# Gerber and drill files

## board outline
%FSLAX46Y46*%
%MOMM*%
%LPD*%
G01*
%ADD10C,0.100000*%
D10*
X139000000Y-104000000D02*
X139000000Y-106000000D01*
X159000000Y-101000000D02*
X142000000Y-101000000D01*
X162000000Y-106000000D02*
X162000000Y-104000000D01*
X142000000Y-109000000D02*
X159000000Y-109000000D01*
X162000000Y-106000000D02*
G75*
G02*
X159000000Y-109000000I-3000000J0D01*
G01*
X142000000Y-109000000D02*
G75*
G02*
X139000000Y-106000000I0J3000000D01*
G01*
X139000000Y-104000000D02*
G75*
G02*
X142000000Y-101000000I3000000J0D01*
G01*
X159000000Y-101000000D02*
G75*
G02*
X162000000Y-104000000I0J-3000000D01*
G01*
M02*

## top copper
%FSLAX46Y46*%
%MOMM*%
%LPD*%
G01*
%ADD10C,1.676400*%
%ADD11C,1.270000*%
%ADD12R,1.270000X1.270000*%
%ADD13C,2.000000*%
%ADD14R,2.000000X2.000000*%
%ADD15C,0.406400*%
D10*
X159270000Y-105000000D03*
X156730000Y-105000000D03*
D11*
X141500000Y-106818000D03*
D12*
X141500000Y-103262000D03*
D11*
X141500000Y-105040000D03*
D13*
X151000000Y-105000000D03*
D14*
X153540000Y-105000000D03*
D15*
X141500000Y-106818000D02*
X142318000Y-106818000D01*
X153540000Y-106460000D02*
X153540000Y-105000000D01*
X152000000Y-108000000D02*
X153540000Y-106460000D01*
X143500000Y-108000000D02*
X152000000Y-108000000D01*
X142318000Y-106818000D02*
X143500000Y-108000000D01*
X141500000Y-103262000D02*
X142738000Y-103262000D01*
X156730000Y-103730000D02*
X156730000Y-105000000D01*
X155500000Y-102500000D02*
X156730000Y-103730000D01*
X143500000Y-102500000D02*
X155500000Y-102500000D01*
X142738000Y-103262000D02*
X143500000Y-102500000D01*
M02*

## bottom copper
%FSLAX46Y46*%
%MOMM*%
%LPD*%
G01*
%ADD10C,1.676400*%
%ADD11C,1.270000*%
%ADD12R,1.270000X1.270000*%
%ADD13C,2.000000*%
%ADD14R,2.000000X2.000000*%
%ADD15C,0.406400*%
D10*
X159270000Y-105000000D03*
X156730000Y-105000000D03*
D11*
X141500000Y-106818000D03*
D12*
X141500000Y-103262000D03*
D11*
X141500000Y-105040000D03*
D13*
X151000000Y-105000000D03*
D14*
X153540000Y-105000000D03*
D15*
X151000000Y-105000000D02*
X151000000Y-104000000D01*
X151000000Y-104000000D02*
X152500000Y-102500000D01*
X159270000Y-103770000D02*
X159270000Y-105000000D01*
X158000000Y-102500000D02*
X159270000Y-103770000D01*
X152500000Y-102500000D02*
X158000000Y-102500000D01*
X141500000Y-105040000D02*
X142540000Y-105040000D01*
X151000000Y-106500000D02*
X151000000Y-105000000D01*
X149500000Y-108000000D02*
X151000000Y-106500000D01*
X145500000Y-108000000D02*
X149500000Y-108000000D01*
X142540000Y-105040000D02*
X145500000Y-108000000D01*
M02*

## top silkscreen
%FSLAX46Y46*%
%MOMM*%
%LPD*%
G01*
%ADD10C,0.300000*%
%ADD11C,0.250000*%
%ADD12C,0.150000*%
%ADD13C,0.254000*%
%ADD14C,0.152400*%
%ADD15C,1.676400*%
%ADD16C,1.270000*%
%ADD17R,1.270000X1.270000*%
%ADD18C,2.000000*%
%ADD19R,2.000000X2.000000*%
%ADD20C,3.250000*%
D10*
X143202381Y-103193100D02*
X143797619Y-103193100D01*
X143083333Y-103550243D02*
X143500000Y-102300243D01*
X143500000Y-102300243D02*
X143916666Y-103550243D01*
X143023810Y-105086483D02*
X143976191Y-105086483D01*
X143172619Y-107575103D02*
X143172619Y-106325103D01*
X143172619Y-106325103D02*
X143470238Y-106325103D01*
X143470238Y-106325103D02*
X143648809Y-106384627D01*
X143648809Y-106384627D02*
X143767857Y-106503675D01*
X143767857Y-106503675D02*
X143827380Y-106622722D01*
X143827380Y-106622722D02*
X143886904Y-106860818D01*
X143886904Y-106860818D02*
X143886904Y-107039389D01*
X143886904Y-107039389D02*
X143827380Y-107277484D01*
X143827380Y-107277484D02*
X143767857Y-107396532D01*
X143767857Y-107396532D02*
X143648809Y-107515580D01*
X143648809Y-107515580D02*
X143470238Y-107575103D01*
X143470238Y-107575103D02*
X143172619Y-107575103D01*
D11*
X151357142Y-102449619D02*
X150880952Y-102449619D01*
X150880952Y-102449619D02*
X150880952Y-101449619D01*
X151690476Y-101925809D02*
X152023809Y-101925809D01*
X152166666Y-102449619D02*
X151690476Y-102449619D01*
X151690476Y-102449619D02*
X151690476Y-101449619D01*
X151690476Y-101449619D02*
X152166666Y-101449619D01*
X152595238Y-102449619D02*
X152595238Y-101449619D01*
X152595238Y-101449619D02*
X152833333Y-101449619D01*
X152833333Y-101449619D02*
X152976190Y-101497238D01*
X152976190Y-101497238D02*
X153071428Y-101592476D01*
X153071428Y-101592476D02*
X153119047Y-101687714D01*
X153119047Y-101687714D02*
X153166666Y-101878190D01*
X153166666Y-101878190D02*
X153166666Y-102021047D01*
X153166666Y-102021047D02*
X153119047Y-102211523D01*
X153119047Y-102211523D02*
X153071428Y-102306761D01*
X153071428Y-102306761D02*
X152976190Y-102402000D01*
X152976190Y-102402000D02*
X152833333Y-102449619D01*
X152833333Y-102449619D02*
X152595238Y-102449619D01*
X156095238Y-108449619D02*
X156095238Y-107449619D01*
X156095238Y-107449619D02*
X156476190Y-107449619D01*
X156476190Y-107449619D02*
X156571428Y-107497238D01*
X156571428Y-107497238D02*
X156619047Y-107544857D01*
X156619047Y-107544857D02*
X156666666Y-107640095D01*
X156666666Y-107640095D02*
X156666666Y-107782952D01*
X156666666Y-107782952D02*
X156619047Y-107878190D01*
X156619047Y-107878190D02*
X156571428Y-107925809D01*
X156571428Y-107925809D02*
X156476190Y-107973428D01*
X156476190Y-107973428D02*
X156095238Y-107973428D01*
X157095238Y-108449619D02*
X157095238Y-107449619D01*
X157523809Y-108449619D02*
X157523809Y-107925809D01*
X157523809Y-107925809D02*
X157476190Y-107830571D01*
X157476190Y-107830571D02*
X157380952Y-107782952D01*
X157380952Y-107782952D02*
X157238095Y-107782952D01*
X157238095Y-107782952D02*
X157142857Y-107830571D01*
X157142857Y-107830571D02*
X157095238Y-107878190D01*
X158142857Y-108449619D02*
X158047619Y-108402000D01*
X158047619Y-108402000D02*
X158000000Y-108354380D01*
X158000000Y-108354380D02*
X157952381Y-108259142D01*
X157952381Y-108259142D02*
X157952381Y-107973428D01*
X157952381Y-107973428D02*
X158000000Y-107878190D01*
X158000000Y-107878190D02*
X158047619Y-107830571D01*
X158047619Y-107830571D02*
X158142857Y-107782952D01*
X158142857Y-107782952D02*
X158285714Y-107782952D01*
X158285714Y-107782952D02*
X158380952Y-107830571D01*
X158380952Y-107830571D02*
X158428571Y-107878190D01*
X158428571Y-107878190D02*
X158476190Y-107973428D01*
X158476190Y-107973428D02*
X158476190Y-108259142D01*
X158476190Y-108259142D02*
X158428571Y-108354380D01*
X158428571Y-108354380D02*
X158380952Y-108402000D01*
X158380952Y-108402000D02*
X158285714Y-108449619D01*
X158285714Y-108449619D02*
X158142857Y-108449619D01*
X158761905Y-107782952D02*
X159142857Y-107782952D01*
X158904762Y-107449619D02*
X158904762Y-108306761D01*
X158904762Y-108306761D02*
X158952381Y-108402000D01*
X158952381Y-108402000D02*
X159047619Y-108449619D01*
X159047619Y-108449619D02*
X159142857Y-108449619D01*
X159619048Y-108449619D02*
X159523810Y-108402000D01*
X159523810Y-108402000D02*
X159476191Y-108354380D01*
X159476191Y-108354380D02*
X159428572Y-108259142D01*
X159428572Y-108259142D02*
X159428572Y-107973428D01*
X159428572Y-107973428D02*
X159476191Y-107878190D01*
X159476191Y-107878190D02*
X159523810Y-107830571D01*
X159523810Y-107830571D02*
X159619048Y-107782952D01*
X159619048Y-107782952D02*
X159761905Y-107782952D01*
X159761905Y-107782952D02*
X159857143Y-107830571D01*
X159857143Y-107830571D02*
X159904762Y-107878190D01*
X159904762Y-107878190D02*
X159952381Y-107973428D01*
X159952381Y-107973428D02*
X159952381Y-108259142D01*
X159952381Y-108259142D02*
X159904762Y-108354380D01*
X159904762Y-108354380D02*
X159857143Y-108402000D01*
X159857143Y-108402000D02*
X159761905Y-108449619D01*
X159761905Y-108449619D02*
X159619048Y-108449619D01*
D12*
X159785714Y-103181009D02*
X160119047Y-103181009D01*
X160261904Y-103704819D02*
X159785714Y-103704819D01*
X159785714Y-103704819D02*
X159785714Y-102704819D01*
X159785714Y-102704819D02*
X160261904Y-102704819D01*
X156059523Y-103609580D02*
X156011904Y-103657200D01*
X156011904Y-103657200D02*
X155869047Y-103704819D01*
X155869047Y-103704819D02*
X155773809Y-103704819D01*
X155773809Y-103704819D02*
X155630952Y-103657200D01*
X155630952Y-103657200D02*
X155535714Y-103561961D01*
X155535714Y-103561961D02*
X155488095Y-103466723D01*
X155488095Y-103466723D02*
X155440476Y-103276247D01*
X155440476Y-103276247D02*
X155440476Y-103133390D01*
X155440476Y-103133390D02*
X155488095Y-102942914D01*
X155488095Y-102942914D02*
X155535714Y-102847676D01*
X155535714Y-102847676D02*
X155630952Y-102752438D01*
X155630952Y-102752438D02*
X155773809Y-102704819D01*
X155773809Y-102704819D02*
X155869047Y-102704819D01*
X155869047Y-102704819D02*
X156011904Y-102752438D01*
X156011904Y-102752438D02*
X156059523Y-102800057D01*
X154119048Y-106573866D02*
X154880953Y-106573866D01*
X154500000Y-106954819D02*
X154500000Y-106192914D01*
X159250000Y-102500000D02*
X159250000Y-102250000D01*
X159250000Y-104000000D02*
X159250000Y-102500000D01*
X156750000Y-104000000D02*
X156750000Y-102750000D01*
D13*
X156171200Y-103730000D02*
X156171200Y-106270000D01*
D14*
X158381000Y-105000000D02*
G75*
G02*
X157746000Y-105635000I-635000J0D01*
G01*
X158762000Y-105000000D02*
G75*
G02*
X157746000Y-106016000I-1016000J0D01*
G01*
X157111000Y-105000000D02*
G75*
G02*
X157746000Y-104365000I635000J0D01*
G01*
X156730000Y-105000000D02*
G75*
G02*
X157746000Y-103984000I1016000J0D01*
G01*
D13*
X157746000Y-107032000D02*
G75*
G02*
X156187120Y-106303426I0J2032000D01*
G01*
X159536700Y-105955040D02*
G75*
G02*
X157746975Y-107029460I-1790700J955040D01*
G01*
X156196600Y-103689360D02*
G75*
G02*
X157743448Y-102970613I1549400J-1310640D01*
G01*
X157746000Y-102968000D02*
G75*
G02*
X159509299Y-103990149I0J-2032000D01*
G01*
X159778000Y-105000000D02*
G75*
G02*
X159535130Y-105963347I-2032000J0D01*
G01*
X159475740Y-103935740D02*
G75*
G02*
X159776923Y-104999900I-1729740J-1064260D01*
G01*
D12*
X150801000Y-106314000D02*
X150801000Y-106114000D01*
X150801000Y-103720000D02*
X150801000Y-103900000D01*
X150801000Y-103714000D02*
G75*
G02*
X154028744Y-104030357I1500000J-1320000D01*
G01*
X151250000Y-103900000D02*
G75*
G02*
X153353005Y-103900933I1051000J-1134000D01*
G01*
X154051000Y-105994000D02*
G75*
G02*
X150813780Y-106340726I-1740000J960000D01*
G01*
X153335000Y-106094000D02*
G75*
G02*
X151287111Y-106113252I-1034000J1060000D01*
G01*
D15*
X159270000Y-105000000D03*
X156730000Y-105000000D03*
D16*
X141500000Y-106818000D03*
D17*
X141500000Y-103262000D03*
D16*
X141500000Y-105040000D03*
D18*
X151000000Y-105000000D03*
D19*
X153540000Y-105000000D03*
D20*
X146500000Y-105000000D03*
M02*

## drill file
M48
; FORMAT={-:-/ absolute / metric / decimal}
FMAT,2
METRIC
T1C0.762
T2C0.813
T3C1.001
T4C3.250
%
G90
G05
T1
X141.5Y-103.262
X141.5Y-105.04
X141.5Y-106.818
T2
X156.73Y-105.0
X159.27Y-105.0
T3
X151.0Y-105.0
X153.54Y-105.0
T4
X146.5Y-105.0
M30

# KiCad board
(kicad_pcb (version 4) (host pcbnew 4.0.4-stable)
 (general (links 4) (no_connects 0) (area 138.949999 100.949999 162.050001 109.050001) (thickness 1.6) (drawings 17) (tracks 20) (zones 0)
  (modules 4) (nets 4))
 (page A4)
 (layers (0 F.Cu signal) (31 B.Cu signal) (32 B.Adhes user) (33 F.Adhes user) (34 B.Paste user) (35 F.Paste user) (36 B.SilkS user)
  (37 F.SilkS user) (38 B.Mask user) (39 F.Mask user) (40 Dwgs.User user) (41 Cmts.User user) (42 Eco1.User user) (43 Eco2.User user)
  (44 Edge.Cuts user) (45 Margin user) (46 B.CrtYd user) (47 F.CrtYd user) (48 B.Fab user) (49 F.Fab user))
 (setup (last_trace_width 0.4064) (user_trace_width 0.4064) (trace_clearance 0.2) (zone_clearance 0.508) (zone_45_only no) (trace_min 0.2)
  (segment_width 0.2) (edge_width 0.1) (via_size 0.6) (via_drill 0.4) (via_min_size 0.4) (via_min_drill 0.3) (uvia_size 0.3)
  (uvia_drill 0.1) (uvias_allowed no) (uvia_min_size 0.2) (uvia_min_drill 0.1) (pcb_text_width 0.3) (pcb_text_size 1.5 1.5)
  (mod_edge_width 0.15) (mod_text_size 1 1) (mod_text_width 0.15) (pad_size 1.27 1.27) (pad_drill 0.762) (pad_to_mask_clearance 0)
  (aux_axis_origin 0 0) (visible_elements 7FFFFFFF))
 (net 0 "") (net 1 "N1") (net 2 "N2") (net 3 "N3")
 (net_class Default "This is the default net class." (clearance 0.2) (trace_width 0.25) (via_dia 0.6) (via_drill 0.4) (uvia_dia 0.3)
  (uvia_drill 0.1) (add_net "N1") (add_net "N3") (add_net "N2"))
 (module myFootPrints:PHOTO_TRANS (layer F.Cu) (at 158 105 180)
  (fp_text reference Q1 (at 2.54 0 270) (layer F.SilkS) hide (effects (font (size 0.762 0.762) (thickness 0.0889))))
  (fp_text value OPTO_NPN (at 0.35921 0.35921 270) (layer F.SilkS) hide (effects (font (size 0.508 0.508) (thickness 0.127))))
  (fp_line (start -1.25 2.5) (end -1.25 2.75) (layer F.SilkS) (width 0.15))
  (fp_line (start -1.25 1) (end -1.25 2.5) (layer F.SilkS) (width 0.15))
  (fp_line (start 1.25 1) (end 1.25 2.25) (layer F.SilkS) (width 0.15))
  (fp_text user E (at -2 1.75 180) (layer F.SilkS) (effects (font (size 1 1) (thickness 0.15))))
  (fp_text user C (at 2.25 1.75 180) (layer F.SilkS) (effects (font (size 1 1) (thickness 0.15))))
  (fp_line (start 1.8288 1.27) (end 1.8288 -1.27) (layer F.SilkS) (width 0.254))
  (fp_arc (start 0.254 0) (end -0.381 0) (angle 90) (layer F.SilkS) (width 0.1524))
  (fp_arc (start 0.254 0) (end -0.762 0) (angle 90) (layer F.SilkS) (width 0.1524))
  (fp_arc (start 0.254 0) (end 0.889 0) (angle 90) (layer F.SilkS) (width 0.1524))
  (fp_arc (start 0.254 0) (end 1.27 0) (angle 90) (layer F.SilkS) (width 0.1524))
  (fp_arc (start 0.254 0) (end 0.254 -2.032) (angle 50.1) (layer F.SilkS) (width 0.254))
  (fp_arc (start 0.254 0) (end -1.5367 -0.95504) (angle 61.9) (layer F.SilkS) (width 0.254))
  (fp_arc (start 0.254 0) (end 1.8034 1.31064) (angle 49.7) (layer F.SilkS) (width 0.254))
  (fp_arc (start 0.254 0) (end 0.254 2.032) (angle 60.2) (layer F.SilkS) (width 0.254))
  (fp_arc (start 0.254 0) (end -1.778 0) (angle 28.3) (layer F.SilkS) (width 0.254))
  (fp_arc (start 0.254 0) (end -1.47574 1.06426) (angle 31.6) (layer F.SilkS) (width 0.254))
  (pad 1 thru_hole circle (at -1.27 0 180) (size 1.6764 1.6764) (drill 0.8128) (layers *.Cu *.Mask F.SilkS) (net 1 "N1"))
  (pad 3 thru_hole circle (at 1.27 0 225) (size 1.6764 1.6764) (drill 0.8128) (layers *.Cu *.Mask F.SilkS) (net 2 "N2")))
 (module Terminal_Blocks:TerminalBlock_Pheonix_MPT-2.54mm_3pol (layer F.Cu) (at 141.5 102.5 270)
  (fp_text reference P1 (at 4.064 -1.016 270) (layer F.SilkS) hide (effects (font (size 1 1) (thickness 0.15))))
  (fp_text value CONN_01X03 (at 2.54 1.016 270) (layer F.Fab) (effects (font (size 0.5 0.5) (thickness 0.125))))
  (pad 3 thru_hole circle (at 4.318 0 270) (size 1.27 1.27) (drill 0.762) (layers *.Cu *.Mask F.SilkS) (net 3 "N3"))
  (pad 1 thru_hole rect (at 0.762 0 270) (size 1.27 1.27) (drill 0.762) (layers *.Cu *.Mask F.SilkS) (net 2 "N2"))
  (pad 2 thru_hole circle (at 2.54 0 270) (size 1.27 1.27) (drill 0.762) (layers *.Cu *.Mask F.SilkS) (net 1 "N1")))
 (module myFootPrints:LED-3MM (layer F.Cu) (at 151 105)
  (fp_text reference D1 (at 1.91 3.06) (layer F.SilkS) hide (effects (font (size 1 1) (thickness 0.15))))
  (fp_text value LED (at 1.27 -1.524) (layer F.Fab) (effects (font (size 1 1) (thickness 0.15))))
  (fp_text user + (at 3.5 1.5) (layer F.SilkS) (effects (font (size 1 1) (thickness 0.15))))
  (fp_line (start -0.199 1.314) (end -0.199 1.114) (layer F.SilkS) (width 0.15))
  (fp_line (start -0.199 -1.28) (end -0.199 -1.1) (layer F.SilkS) (width 0.15))
  (fp_arc (start 1.301 0.034) (end -0.199 -1.286) (angle 108.5) (layer F.SilkS) (width 0.15))
  (fp_arc (start 1.301 0.034) (end 0.25 -1.1) (angle 85.7) (layer F.SilkS) (width 0.15))
  (fp_arc (start 1.311 0.034) (end 3.051 0.994) (angle 110) (layer F.SilkS) (width 0.15))
  (fp_arc (start 1.301 0.034) (end 2.335 1.094) (angle 87.5) (layer F.SilkS) (width 0.15))
  (pad 1 thru_hole circle (at 0 0 90) (size 2 2) (drill 1.00076) (layers *.Cu *.Mask F.SilkS) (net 1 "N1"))
  (pad 2 thru_hole rect (at 2.54 0) (size 2 2) (drill 1.00076) (layers *.Cu *.Mask F.SilkS) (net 3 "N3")))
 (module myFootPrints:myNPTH (layer F.Cu) (at 146.5 105)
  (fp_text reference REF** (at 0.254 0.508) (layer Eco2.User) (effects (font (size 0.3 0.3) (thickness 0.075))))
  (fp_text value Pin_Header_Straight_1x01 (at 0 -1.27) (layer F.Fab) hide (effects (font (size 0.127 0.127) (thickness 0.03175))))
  (pad "" np_thru_hole circle (at 0 0) (size 3.25 3.25) (drill 3.25) (layers *.Cu *.Mask F.SilkS) (thermal_width 4) (thermal_gap 4)))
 (gr_line (start 139 104) (end 139 106) (angle 90) (layer Edge.Cuts) (width 0.1))
 (gr_line (start 159 101) (end 142 101) (angle 90) (layer Edge.Cuts) (width 0.1))
 (gr_line (start 162 106) (end 162 104) (angle 90) (layer Edge.Cuts) (width 0.1))
 (gr_line (start 142 109) (end 159 109) (angle 90) (layer Edge.Cuts) (width 0.1))
 (gr_arc (start 159 106) (end 162 106) (angle 90) (layer Edge.Cuts) (width 0.1))
 (gr_arc (start 142 106) (end 142 109) (angle 90) (layer Edge.Cuts) (width 0.1))
 (gr_arc (start 142 104) (end 139 104) (angle 90) (layer Edge.Cuts) (width 0.1))
 (gr_arc (start 159 104) (end 159 101) (angle 90) (layer Edge.Cuts) (width 0.1))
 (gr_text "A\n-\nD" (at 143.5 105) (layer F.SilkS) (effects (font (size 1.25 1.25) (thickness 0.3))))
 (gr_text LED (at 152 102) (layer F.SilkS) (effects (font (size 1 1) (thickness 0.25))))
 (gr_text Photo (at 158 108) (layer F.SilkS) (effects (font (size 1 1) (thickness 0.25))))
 (segment (start 151 105) (end 151 104) (width 0.4064) (layer B.Cu) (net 1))
 (segment (start 151 104) (end 152.5 102.5) (width 0.4064) (layer B.Cu) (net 1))
 (segment (start 159.27 103.77) (end 159.27 105) (width 0.4064) (layer B.Cu) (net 1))
 (segment (start 158 102.5) (end 159.27 103.77) (width 0.4064) (layer B.Cu) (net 1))
 (segment (start 152.5 102.5) (end 158 102.5) (width 0.4064) (layer B.Cu) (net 1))
 (segment (start 141.5 105.04) (end 142.54 105.04) (width 0.4064) (layer B.Cu) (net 1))
 (segment (start 151 106.5) (end 151 105) (width 0.4064) (layer B.Cu) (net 1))
 (segment (start 149.5 108) (end 151 106.5) (width 0.4064) (layer B.Cu) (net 1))
 (segment (start 145.5 108) (end 149.5 108) (width 0.4064) (layer B.Cu) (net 1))
 (segment (start 142.54 105.04) (end 145.5 108) (width 0.4064) (layer B.Cu) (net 1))
 (segment (start 141.5 106.818) (end 142.318 106.818) (width 0.4064) (layer F.Cu) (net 3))
 (segment (start 153.54 106.46) (end 153.54 105) (width 0.4064) (layer F.Cu) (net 3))
 (segment (start 152 108) (end 153.54 106.46) (width 0.4064) (layer F.Cu) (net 3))
 (segment (start 143.5 108) (end 152 108) (width 0.4064) (layer F.Cu) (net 3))
 (segment (start 142.318 106.818) (end 143.5 108) (width 0.4064) (layer F.Cu) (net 3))
 (segment (start 141.5 103.262) (end 142.738 103.262) (width 0.4064) (layer F.Cu) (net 2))
 (segment (start 156.73 103.73) (end 156.73 105) (width 0.4064) (layer F.Cu) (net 2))
 (segment (start 155.5 102.5) (end 156.73 103.73) (width 0.4064) (layer F.Cu) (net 2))
 (segment (start 143.5 102.5) (end 155.5 102.5) (width 0.4064) (layer F.Cu) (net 2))
 (segment (start 142.738 103.262) (end 143.5 102.5) (width 0.4064) (layer F.Cu) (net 2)))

